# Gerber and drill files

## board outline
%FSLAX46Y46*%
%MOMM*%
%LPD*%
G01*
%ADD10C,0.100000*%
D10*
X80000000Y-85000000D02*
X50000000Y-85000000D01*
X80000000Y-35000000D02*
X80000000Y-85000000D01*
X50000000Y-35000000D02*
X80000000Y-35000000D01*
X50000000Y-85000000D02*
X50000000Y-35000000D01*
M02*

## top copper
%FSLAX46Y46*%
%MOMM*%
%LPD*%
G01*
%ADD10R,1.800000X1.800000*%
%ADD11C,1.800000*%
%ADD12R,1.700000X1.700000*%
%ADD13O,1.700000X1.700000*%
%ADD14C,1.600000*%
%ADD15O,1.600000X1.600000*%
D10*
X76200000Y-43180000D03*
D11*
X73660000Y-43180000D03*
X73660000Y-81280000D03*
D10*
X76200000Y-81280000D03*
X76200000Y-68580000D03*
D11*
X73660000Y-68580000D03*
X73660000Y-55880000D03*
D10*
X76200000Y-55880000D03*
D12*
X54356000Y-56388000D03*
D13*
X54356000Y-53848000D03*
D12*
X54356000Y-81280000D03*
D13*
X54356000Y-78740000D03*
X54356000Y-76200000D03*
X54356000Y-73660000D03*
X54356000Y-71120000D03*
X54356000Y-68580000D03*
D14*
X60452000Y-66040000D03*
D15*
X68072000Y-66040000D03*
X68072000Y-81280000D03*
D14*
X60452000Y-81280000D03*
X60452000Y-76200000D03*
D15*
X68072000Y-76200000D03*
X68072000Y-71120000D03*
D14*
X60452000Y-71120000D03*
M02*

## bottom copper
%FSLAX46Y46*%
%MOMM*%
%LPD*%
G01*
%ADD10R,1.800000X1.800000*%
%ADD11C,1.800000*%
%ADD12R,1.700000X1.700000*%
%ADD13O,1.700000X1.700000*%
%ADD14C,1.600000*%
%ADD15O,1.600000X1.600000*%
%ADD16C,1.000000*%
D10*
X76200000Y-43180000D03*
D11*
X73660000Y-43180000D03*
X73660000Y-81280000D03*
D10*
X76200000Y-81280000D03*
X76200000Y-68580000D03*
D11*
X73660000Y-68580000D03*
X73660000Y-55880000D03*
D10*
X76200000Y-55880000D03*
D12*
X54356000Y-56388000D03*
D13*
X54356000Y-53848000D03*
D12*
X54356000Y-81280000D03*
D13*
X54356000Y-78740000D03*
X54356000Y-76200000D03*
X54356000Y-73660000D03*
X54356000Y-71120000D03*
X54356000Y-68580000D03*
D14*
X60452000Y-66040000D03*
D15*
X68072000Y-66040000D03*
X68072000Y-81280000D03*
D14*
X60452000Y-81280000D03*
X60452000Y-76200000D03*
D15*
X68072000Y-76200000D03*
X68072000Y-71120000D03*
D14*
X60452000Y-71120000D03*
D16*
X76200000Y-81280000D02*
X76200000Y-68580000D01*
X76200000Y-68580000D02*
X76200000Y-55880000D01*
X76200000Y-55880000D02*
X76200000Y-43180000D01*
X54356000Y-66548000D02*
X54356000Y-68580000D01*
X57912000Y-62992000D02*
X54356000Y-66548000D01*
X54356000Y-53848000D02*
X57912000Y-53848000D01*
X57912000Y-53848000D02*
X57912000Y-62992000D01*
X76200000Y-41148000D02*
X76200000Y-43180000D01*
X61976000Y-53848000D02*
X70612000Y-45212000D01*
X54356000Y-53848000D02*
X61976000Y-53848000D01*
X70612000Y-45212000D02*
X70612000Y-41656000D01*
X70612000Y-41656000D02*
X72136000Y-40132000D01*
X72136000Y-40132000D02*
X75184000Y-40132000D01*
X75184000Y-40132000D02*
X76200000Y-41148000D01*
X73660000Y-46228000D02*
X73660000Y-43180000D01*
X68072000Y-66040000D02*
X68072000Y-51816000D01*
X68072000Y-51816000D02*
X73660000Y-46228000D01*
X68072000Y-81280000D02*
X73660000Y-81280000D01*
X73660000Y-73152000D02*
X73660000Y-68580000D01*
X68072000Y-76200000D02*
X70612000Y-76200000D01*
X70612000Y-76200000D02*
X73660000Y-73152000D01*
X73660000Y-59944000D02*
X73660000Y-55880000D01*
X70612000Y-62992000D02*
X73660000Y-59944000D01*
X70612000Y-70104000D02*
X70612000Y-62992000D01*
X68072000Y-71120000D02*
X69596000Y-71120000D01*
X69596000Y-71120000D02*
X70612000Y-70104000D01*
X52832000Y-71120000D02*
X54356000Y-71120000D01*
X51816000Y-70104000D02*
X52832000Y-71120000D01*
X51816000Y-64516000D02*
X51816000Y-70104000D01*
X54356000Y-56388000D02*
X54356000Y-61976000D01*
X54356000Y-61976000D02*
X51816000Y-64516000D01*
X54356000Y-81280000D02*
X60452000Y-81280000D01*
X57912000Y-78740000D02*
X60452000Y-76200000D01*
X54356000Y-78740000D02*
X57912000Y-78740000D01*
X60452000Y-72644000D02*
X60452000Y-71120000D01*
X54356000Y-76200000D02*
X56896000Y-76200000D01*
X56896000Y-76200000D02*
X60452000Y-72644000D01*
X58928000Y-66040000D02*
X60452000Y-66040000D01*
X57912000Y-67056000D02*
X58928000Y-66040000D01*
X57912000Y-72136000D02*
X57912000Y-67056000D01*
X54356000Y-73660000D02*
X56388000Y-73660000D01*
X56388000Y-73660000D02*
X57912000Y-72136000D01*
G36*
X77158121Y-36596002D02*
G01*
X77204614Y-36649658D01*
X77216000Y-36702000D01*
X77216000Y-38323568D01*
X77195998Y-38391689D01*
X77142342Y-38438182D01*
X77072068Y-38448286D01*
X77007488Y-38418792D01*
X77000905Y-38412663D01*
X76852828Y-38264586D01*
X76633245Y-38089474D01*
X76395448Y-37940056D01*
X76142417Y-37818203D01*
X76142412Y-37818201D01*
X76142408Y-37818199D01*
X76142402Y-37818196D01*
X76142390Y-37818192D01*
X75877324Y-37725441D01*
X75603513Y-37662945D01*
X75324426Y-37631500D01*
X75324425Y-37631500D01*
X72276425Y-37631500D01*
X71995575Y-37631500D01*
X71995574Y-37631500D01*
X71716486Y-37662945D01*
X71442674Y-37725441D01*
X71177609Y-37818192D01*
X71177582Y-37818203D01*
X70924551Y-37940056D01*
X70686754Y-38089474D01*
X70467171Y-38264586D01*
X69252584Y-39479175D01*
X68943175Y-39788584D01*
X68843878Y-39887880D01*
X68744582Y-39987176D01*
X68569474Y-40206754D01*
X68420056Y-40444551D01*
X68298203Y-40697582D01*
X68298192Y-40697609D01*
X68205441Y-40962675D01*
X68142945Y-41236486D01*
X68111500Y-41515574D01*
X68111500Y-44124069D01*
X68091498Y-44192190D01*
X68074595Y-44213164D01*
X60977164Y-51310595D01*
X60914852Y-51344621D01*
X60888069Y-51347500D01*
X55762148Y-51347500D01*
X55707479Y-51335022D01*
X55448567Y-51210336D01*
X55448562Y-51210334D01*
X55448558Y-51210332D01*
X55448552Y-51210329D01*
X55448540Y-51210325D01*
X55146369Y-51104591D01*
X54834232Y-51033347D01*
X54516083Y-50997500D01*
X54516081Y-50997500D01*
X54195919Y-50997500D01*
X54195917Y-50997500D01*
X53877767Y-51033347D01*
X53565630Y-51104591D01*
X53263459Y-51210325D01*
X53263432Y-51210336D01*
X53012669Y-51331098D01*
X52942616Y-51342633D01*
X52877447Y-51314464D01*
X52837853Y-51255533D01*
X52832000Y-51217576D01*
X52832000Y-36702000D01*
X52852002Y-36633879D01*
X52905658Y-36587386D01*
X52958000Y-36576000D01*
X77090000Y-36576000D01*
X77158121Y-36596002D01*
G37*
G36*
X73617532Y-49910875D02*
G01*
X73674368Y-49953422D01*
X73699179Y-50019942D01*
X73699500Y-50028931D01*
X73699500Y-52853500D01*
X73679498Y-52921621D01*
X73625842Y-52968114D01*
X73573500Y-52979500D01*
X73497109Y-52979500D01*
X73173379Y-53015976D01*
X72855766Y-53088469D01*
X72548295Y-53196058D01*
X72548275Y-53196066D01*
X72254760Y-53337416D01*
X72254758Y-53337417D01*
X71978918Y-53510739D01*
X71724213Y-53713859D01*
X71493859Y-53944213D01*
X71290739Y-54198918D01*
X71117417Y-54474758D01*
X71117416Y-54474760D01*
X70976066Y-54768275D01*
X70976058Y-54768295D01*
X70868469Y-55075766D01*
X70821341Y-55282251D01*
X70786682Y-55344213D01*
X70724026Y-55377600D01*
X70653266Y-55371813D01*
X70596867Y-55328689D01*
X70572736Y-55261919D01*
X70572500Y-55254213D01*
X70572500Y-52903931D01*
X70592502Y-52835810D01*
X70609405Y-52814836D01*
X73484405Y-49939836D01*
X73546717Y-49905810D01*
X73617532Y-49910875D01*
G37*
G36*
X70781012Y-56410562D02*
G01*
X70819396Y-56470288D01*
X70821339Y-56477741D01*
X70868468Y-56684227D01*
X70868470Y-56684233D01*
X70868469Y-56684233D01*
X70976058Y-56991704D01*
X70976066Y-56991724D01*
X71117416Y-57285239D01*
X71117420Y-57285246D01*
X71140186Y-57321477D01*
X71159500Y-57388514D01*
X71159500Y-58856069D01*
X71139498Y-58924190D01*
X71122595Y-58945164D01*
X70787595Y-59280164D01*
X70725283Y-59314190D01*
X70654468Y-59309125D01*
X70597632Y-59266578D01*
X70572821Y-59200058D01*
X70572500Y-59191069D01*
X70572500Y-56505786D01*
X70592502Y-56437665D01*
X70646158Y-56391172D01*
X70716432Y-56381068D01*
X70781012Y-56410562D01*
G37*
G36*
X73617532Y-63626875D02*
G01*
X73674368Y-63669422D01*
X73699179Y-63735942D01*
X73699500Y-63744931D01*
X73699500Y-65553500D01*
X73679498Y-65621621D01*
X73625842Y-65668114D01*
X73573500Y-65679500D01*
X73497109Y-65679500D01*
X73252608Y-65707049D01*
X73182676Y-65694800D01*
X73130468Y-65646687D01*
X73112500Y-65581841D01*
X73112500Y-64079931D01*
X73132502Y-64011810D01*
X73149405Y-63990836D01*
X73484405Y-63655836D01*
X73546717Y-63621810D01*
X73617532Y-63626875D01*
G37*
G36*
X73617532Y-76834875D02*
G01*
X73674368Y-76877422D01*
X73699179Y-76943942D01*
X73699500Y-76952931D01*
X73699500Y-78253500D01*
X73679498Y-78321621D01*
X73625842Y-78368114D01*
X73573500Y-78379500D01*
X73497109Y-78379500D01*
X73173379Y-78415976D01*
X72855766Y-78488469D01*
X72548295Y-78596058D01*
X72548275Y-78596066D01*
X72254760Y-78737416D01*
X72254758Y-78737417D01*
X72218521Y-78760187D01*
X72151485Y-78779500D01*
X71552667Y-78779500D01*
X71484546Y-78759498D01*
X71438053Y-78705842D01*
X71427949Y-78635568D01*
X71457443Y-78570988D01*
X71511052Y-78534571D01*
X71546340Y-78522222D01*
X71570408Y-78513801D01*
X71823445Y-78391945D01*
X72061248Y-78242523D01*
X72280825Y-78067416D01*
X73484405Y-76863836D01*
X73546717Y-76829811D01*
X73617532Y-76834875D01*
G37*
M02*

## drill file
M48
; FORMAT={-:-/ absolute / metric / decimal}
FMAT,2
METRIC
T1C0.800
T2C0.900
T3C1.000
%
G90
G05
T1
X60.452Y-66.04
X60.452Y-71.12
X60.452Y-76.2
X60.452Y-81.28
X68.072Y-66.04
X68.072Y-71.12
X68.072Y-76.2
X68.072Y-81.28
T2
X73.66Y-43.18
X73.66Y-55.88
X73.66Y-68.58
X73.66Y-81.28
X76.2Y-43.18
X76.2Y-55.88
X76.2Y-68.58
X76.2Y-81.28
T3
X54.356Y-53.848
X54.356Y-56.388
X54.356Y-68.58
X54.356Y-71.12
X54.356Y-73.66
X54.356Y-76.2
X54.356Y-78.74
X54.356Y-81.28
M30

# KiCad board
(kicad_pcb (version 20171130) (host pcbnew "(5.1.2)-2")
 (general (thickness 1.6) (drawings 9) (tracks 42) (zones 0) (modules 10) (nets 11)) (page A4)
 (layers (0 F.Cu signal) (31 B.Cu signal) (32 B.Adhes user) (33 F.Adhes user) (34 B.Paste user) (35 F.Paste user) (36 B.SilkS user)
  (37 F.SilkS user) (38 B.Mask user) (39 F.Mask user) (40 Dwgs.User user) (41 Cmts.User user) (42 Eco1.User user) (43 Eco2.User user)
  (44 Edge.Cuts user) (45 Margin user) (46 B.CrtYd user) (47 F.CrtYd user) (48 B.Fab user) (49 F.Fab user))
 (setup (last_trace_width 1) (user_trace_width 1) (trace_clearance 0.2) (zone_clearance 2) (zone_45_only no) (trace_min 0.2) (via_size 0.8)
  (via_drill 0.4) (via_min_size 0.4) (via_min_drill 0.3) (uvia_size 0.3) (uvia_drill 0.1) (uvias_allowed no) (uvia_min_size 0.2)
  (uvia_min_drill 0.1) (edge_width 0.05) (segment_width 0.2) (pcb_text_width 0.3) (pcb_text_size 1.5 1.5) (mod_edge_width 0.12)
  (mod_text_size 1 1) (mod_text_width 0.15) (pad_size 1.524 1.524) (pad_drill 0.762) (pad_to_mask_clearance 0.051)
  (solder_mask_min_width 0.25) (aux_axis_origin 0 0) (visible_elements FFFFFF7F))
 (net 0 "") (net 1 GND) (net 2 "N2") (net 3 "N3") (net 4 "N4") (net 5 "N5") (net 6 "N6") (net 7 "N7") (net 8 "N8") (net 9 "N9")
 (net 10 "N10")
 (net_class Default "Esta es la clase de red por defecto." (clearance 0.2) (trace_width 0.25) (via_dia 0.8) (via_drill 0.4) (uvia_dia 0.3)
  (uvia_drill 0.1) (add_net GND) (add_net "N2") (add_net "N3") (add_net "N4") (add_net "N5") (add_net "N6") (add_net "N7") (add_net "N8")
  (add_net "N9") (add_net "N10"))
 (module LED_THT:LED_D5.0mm (layer F.Cu) (at 76.2 43.18 180)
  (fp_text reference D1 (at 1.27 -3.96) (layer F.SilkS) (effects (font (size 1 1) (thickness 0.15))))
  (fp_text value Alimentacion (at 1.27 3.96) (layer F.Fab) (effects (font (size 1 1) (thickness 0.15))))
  (pad 1 thru_hole rect (at 0 0 180) (size 1.8 1.8) (drill 0.9) (layers *.Cu *.Mask) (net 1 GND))
  (pad 2 thru_hole circle (at 2.54 0 180) (size 1.8 1.8) (drill 0.9) (layers *.Cu *.Mask) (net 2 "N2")))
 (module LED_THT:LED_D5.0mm (layer F.Cu) (at 76.2 81.28 180)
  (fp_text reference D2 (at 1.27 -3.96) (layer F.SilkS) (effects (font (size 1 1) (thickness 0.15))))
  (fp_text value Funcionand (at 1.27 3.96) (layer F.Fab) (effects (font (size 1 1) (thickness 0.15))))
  (pad 2 thru_hole circle (at 2.54 0 180) (size 1.8 1.8) (drill 0.9) (layers *.Cu *.Mask) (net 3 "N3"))
  (pad 1 thru_hole rect (at 0 0 180) (size 1.8 1.8) (drill 0.9) (layers *.Cu *.Mask) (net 1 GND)))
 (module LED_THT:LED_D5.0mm (layer F.Cu) (at 76.2 68.58 180)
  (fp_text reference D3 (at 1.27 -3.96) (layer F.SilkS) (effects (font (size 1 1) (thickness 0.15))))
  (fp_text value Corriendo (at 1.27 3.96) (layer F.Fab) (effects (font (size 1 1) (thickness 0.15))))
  (pad 1 thru_hole rect (at 0 0 180) (size 1.8 1.8) (drill 0.9) (layers *.Cu *.Mask) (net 1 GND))
  (pad 2 thru_hole circle (at 2.54 0 180) (size 1.8 1.8) (drill 0.9) (layers *.Cu *.Mask) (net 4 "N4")))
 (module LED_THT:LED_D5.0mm (layer F.Cu) (at 76.2 55.88 180)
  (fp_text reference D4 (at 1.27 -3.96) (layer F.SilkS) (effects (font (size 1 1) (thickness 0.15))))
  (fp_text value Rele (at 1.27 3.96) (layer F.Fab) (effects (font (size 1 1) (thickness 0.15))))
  (pad 2 thru_hole circle (at 2.54 0 180) (size 1.8 1.8) (drill 0.9) (layers *.Cu *.Mask) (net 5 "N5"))
  (pad 1 thru_hole rect (at 0 0 180) (size 1.8 1.8) (drill 0.9) (layers *.Cu *.Mask) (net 1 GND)))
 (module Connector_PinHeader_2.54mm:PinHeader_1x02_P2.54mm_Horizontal (layer F.Cu) (at 54.356 56.388 180)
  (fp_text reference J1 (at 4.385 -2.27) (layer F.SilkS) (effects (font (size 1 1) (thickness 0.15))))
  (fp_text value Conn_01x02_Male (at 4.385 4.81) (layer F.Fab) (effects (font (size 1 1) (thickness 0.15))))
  (pad 1 thru_hole rect (at 0 0 180) (size 1.7 1.7) (drill 1) (layers *.Cu *.Mask) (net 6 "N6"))
  (pad 2 thru_hole oval (at 0 2.54 180) (size 1.7 1.7) (drill 1) (layers *.Cu *.Mask) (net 1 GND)))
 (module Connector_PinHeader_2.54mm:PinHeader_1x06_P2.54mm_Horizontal (layer F.Cu) (at 54.356 81.28 180)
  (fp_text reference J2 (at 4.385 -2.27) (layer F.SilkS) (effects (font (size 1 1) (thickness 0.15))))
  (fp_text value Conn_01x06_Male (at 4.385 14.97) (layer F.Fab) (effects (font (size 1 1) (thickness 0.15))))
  (pad 1 thru_hole rect (at 0 0 180) (size 1.7 1.7) (drill 1) (layers *.Cu *.Mask) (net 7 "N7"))
  (pad 2 thru_hole oval (at 0 2.54 180) (size 1.7 1.7) (drill 1) (layers *.Cu *.Mask) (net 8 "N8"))
  (pad 3 thru_hole oval (at 0 5.08 180) (size 1.7 1.7) (drill 1) (layers *.Cu *.Mask) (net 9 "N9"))
  (pad 4 thru_hole oval (at 0 7.62 180) (size 1.7 1.7) (drill 1) (layers *.Cu *.Mask) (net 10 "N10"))
  (pad 5 thru_hole oval (at 0 10.16 180) (size 1.7 1.7) (drill 1) (layers *.Cu *.Mask) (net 6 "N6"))
  (pad 6 thru_hole oval (at 0 12.7 180) (size 1.7 1.7) (drill 1) (layers *.Cu *.Mask) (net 1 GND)))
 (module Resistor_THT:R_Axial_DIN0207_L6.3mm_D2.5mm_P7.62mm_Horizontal (layer F.Cu) (at 60.452 66.04)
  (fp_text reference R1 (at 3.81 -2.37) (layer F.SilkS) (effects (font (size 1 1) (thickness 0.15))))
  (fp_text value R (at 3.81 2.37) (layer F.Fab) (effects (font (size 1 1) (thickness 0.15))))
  (pad 1 thru_hole circle (at 0 0) (size 1.6 1.6) (drill 0.8) (layers *.Cu *.Mask) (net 10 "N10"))
  (pad 2 thru_hole oval (at 7.62 0) (size 1.6 1.6) (drill 0.8) (layers *.Cu *.Mask) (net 2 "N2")))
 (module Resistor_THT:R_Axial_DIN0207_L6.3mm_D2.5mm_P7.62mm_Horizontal (layer F.Cu) (at 60.452 81.28)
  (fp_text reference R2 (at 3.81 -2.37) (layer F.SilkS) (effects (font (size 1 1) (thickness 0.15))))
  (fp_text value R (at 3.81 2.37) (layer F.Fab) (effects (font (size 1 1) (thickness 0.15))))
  (pad 2 thru_hole oval (at 7.62 0) (size 1.6 1.6) (drill 0.8) (layers *.Cu *.Mask) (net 3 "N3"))
  (pad 1 thru_hole circle (at 0 0) (size 1.6 1.6) (drill 0.8) (layers *.Cu *.Mask) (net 7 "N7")))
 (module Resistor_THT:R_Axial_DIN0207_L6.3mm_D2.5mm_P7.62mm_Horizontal (layer F.Cu) (at 60.452 76.2)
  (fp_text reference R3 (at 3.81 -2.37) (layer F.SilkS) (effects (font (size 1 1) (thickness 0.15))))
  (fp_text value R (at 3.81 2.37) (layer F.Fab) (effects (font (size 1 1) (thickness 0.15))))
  (pad 1 thru_hole circle (at 0 0) (size 1.6 1.6) (drill 0.8) (layers *.Cu *.Mask) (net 8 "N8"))
  (pad 2 thru_hole oval (at 7.62 0) (size 1.6 1.6) (drill 0.8) (layers *.Cu *.Mask) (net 4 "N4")))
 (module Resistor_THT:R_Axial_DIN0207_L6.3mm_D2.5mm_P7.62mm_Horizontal (layer F.Cu) (at 60.452 71.12)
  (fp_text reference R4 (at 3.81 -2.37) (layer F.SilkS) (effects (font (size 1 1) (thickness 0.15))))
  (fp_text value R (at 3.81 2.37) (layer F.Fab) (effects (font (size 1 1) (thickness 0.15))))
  (pad 2 thru_hole oval (at 7.62 0) (size 1.6 1.6) (drill 0.8) (layers *.Cu *.Mask) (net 5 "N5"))
  (pad 1 thru_hole circle (at 0 0) (size 1.6 1.6) (drill 0.8) (layers *.Cu *.Mask) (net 9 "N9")))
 (gr_line (start 80 85) (end 50 85) (layer Edge.Cuts) (width 0.1))
 (gr_line (start 80 35) (end 80 85) (layer Edge.Cuts) (width 0.1))
 (gr_line (start 50 35) (end 80 35) (layer Edge.Cuts) (width 0.1))
 (gr_line (start 50 85) (end 50 35) (layer Edge.Cuts) (width 0.1))
 (segment (start 76.2 81.28) (end 76.2 68.58) (width 1) (layer B.Cu) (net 1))
 (segment (start 76.2 68.58) (end 76.2 55.88) (width 1) (layer B.Cu) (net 1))
 (segment (start 76.2 55.88) (end 76.2 43.18) (width 1) (layer B.Cu) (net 1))
 (segment (start 54.356 66.548) (end 54.356 68.58) (width 1) (layer B.Cu) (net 1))
 (segment (start 57.912 62.992) (end 54.356 66.548) (width 1) (layer B.Cu) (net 1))
 (segment (start 54.356 53.848) (end 57.912 53.848) (width 1) (layer B.Cu) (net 1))
 (segment (start 57.912 53.848) (end 57.912 62.992) (width 1) (layer B.Cu) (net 1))
 (segment (start 76.2 41.148) (end 76.2 43.18) (width 1) (layer B.Cu) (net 1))
 (segment (start 61.976 53.848) (end 70.612 45.212) (width 1) (layer B.Cu) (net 1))
 (segment (start 54.356 53.848) (end 61.976 53.848) (width 1) (layer B.Cu) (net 1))
 (segment (start 70.612 45.212) (end 70.612 41.656) (width 1) (layer B.Cu) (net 1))
 (segment (start 70.612 41.656) (end 72.136 40.132) (width 1) (layer B.Cu) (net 1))
 (segment (start 72.136 40.132) (end 75.184 40.132) (width 1) (layer B.Cu) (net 1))
 (segment (start 75.184 40.132) (end 76.2 41.148) (width 1) (layer B.Cu) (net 1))
 (segment (start 73.66 46.228) (end 73.66 43.18) (width 1) (layer B.Cu) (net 2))
 (segment (start 68.072 66.04) (end 68.072 51.816) (width 1) (layer B.Cu) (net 2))
 (segment (start 68.072 51.816) (end 73.66 46.228) (width 1) (layer B.Cu) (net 2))
 (segment (start 68.072 81.28) (end 73.66 81.28) (width 1) (layer B.Cu) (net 3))
 (segment (start 73.66 73.152) (end 73.66 68.58) (width 1) (layer B.Cu) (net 4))
 (segment (start 68.072 76.2) (end 70.612 76.2) (width 1) (layer B.Cu) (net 4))
 (segment (start 70.612 76.2) (end 73.66 73.152) (width 1) (layer B.Cu) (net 4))
 (segment (start 73.66 59.944) (end 73.66 55.88) (width 1) (layer B.Cu) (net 5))
 (segment (start 70.612 62.992) (end 73.66 59.944) (width 1) (layer B.Cu) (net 5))
 (segment (start 70.612 70.104) (end 70.612 62.992) (width 1) (layer B.Cu) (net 5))
 (segment (start 68.072 71.12) (end 69.596 71.12) (width 1) (layer B.Cu) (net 5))
 (segment (start 69.596 71.12) (end 70.612 70.104) (width 1) (layer B.Cu) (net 5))
 (segment (start 52.832 71.12) (end 54.356 71.12) (width 1) (layer B.Cu) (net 6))
 (segment (start 51.816 70.104) (end 52.832 71.12) (width 1) (layer B.Cu) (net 6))
 (segment (start 51.816 64.516) (end 51.816 70.104) (width 1) (layer B.Cu) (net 6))
 (segment (start 54.356 56.388) (end 54.356 61.976) (width 1) (layer B.Cu) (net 6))
 (segment (start 54.356 61.976) (end 51.816 64.516) (width 1) (layer B.Cu) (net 6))
 (segment (start 54.356 81.28) (end 60.452 81.28) (width 1) (layer B.Cu) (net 7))
 (segment (start 57.912 78.74) (end 60.452 76.2) (width 1) (layer B.Cu) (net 8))
 (segment (start 54.356 78.74) (end 57.912 78.74) (width 1) (layer B.Cu) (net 8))
 (segment (start 60.452 72.644) (end 60.452 71.12) (width 1) (layer B.Cu) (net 9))
 (segment (start 54.356 76.2) (end 56.896 76.2) (width 1) (layer B.Cu) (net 9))
 (segment (start 56.896 76.2) (end 60.452 72.644) (width 1) (layer B.Cu) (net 9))
 (segment (start 58.928 66.04) (end 60.452 66.04) (width 1) (layer B.Cu) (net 10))
 (segment (start 57.912 67.056) (end 58.928 66.04) (width 1) (layer B.Cu) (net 10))
 (segment (start 57.912 72.136) (end 57.912 67.056) (width 1) (layer B.Cu) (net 10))
 (segment (start 54.356 73.66) (end 56.388 73.66) (width 1) (layer B.Cu) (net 10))
 (segment (start 56.388 73.66) (end 57.912 72.136) (width 1) (layer B.Cu) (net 10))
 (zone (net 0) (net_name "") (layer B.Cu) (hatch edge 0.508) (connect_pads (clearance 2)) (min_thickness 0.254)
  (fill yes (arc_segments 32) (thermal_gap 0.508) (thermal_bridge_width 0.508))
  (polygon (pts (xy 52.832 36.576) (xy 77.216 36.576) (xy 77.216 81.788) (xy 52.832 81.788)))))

